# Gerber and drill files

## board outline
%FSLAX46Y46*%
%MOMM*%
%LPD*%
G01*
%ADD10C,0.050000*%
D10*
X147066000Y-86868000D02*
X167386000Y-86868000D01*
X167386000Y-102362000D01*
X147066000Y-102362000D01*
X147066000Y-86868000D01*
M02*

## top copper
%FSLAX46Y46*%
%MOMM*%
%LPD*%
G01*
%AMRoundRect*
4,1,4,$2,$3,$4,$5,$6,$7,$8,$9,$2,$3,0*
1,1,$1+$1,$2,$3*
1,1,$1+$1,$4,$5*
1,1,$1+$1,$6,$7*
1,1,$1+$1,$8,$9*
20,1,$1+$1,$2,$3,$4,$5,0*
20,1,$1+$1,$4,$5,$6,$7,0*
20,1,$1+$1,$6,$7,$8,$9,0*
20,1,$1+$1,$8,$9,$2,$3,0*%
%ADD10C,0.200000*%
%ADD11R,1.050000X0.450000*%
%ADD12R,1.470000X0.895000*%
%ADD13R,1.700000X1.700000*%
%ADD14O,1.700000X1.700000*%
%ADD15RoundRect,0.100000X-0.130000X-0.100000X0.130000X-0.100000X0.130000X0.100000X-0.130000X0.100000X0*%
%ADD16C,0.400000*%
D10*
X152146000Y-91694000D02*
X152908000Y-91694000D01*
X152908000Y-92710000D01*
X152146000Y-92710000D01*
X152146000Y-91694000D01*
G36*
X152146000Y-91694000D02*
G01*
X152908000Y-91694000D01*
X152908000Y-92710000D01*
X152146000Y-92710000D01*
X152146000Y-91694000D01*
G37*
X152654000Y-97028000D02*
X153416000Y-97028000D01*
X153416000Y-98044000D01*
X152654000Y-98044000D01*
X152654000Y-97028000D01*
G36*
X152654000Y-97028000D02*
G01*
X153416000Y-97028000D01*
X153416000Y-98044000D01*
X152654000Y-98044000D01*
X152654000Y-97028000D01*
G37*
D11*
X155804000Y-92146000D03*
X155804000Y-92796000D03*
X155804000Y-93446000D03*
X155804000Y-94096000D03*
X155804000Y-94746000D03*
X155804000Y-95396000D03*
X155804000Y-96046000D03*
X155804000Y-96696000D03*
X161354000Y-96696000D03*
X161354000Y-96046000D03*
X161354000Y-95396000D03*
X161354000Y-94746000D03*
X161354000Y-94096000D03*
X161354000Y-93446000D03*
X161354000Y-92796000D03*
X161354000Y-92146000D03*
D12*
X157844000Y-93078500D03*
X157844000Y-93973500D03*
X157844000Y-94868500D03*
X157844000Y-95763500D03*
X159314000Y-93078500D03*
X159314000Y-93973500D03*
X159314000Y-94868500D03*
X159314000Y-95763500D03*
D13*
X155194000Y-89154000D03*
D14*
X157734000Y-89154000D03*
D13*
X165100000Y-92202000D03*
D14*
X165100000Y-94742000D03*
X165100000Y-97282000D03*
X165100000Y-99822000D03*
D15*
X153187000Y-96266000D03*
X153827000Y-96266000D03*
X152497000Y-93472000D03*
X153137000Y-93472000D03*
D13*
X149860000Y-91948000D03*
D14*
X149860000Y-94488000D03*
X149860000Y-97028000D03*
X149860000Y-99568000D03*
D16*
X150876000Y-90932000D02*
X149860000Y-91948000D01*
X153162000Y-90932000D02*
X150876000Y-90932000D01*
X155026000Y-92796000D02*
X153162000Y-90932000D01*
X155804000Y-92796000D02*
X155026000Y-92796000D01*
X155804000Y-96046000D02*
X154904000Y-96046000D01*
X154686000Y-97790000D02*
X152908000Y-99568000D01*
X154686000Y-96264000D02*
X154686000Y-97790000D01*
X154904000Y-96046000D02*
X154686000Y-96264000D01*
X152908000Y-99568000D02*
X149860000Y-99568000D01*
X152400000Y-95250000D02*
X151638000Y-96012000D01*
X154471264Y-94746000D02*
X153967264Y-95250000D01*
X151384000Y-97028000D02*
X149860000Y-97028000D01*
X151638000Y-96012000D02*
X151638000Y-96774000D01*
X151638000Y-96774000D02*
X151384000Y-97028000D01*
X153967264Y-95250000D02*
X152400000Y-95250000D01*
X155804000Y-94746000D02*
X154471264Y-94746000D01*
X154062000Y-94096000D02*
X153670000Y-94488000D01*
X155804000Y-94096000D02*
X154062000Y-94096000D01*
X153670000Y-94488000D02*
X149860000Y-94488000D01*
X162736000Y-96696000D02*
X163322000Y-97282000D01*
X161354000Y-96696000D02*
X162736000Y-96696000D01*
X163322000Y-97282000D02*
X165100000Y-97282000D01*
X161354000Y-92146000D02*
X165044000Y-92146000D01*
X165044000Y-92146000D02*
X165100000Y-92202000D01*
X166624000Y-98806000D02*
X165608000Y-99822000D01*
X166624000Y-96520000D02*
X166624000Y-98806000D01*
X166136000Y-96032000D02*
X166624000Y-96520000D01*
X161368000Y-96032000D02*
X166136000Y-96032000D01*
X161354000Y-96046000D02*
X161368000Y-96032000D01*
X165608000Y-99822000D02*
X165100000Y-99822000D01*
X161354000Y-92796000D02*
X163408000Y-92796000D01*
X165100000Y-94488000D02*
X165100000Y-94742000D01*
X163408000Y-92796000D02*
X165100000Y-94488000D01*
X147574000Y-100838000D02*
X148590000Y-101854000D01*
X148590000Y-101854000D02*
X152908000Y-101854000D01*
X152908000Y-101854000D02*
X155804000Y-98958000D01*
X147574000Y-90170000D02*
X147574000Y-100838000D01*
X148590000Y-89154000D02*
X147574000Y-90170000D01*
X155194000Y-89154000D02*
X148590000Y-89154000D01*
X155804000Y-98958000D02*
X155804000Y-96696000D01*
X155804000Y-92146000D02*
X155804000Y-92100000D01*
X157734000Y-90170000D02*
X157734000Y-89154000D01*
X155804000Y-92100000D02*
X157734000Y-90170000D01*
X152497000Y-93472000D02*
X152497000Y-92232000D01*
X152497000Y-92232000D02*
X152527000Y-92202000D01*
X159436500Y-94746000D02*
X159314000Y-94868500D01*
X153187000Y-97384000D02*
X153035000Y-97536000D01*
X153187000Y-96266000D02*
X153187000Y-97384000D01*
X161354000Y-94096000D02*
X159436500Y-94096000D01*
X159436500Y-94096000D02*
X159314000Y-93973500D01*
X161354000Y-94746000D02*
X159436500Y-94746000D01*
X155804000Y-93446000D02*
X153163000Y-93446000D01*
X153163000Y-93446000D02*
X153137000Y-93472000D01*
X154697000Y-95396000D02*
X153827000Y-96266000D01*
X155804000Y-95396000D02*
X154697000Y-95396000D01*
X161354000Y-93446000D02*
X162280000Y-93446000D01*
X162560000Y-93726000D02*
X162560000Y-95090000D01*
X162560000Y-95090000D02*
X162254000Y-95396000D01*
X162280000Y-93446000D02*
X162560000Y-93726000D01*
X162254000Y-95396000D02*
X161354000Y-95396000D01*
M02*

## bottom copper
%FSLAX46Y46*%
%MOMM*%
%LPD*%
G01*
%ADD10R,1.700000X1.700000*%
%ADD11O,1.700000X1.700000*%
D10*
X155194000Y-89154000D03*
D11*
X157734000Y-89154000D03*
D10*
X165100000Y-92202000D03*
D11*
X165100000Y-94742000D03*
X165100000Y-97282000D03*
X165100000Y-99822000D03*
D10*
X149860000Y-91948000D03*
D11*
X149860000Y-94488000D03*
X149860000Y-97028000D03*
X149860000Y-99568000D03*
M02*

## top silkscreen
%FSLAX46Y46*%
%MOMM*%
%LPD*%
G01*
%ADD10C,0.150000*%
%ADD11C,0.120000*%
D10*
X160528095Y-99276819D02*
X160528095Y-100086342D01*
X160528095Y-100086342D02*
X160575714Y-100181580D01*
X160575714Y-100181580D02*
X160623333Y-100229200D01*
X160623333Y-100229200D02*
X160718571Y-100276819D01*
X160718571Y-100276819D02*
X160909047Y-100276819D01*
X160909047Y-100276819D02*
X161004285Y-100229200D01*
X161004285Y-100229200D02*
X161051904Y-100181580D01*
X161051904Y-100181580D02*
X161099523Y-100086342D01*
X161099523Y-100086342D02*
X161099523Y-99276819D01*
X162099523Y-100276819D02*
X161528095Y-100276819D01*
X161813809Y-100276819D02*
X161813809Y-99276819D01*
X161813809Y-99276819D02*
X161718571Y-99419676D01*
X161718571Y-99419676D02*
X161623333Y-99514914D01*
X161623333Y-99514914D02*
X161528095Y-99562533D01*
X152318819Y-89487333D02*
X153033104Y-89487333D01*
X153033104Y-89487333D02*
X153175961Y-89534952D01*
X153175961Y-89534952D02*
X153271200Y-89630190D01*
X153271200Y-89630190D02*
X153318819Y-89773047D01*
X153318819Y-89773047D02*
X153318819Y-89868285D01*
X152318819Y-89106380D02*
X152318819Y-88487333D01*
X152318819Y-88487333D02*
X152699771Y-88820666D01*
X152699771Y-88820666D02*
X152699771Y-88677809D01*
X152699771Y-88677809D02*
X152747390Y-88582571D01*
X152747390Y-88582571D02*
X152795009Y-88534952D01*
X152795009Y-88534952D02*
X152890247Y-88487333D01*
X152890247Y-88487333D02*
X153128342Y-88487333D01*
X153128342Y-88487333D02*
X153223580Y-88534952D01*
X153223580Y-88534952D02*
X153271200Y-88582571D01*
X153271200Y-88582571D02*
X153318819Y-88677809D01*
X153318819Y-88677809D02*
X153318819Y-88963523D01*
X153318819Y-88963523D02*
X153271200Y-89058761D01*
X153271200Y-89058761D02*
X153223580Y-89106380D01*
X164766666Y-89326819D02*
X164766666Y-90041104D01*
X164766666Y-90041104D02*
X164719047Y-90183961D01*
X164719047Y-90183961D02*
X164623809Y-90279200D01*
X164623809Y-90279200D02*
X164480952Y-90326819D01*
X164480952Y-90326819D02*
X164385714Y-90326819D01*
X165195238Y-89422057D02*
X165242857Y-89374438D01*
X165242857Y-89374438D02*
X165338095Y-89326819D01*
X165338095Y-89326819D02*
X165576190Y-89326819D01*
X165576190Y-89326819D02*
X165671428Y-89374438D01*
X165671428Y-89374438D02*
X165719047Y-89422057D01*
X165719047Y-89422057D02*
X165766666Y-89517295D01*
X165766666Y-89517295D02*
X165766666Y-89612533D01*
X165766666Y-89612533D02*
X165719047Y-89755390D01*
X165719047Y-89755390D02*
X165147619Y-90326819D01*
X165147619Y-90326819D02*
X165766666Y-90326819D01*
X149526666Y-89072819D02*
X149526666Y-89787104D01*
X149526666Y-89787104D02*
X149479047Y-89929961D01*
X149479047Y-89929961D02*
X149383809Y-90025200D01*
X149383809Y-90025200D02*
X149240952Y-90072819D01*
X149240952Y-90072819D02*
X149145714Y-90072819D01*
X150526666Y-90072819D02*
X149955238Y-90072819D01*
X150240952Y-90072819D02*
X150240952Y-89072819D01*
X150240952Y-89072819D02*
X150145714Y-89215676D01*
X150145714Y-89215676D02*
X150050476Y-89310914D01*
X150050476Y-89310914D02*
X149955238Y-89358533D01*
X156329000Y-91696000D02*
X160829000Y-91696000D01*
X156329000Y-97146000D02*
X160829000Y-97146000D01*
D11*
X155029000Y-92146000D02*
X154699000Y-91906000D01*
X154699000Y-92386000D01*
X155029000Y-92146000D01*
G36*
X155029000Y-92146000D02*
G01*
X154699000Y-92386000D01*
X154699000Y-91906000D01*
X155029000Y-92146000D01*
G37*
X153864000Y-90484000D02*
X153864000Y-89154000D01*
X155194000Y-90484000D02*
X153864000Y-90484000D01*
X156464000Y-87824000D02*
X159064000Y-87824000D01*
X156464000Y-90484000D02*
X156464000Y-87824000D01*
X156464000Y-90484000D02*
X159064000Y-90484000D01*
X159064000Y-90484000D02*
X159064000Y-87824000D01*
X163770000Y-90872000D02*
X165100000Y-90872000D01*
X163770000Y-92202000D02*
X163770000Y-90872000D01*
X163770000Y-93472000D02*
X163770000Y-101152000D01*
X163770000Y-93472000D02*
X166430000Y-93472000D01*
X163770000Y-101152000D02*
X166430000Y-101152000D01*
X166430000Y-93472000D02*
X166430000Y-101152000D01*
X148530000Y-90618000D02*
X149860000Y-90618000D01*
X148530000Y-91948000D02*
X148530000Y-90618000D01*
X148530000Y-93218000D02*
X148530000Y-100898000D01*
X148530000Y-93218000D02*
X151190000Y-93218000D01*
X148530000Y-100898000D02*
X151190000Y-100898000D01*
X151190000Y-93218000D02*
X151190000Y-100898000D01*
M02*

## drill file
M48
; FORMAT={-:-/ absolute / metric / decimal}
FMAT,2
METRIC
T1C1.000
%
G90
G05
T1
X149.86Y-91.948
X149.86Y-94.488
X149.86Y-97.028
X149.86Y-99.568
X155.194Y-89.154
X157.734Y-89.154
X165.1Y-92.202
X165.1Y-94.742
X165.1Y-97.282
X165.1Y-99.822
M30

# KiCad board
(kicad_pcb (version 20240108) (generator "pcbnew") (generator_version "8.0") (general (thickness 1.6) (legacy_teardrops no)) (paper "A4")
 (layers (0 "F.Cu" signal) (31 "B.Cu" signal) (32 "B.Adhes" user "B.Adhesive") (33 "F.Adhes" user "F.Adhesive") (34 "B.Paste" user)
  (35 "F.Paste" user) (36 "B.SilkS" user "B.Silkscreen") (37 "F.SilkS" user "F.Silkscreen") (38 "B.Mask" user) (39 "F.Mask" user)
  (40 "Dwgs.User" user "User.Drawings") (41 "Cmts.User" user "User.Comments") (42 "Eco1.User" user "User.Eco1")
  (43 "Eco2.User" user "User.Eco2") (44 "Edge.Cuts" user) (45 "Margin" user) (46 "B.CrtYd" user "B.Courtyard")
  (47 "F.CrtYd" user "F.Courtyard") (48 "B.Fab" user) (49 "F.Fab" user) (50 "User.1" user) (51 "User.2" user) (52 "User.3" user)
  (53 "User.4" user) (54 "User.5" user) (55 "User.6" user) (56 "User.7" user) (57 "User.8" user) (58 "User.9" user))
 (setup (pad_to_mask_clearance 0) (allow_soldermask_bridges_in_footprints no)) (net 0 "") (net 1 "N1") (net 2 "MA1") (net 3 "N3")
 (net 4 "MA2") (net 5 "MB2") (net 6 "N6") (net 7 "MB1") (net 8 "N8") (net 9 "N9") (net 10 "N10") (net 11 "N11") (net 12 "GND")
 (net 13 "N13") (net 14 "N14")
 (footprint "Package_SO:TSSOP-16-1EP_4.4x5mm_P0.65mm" (layer "F.Cu") (at 158.579 94.421)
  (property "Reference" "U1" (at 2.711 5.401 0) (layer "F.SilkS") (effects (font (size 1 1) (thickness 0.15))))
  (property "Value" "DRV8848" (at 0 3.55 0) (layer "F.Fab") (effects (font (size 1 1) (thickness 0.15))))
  (fp_line (start -2.25 -2.725) (end 2.25 -2.725) (stroke (width 0.15) (type solid)) (layer "F.SilkS"))
  (fp_line (start -2.25 2.725) (end 2.25 2.725) (stroke (width 0.15) (type solid)) (layer "F.SilkS"))
  (fp_poly
   (pts (xy -3.55 -2.275) (xy -3.88 -2.515) (xy -3.88 -2.035) (xy -3.55 -2.275)) (stroke (width 0.12) (type solid)) (fill solid)
   (layer "F.SilkS"))
  (pad "1" smd rect (at -2.775 -2.275) (size 1.05 0.45) (layers "F.Cu" "F.Paste" "F.Mask") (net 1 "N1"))
  (pad "2" smd rect (at -2.775 -1.625) (size 1.05 0.45) (layers "F.Cu" "F.Paste" "F.Mask") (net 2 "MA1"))
  (pad "3" smd rect (at -2.775 -0.975) (size 1.05 0.45) (layers "F.Cu" "F.Paste" "F.Mask") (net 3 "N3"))
  (pad "4" smd rect (at -2.775 -0.325) (size 1.05 0.45) (layers "F.Cu" "F.Paste" "F.Mask") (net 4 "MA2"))
  (pad "5" smd rect (at -2.775 0.325) (size 1.05 0.45) (layers "F.Cu" "F.Paste" "F.Mask") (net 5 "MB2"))
  (pad "6" smd rect (at -2.775 0.975) (size 1.05 0.45) (layers "F.Cu" "F.Paste" "F.Mask") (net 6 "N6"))
  (pad "7" smd rect (at -2.775 1.625) (size 1.05 0.45) (layers "F.Cu" "F.Paste" "F.Mask") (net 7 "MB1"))
  (pad "8" smd rect (at -2.775 2.275) (size 1.05 0.45) (layers "F.Cu" "F.Paste" "F.Mask") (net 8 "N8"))
  (pad "9" smd rect (at 2.775 2.275) (size 1.05 0.45) (layers "F.Cu" "F.Paste" "F.Mask") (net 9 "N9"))
  (pad "10" smd rect (at 2.775 1.625) (size 1.05 0.45) (layers "F.Cu" "F.Paste" "F.Mask") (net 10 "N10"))
  (pad "11" smd rect (at 2.775 0.975) (size 1.05 0.45) (layers "F.Cu" "F.Paste" "F.Mask") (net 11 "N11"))
  (pad "12" smd rect (at 2.775 0.325) (size 1.05 0.45) (layers "F.Cu" "F.Paste" "F.Mask") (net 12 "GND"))
  (pad "13" smd rect (at 2.775 -0.325) (size 1.05 0.45) (layers "F.Cu" "F.Paste" "F.Mask") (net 12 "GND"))
  (pad "14" smd rect (at 2.775 -0.975) (size 1.05 0.45) (layers "F.Cu" "F.Paste" "F.Mask") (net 11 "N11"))
  (pad "15" smd rect (at 2.775 -1.625) (size 1.05 0.45) (layers "F.Cu" "F.Paste" "F.Mask") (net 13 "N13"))
  (pad "16" smd rect (at 2.775 -2.275) (size 1.05 0.45) (layers "F.Cu" "F.Paste" "F.Mask") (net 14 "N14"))
  (pad "17" smd rect (at -0.735 -1.3425) (size 1.47 0.895) (layers "F.Cu" "F.Paste" "F.Mask") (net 12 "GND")
   (solder_paste_margin_ratio -0.2))
  (pad "17" smd rect (at -0.735 -0.4475) (size 1.47 0.895) (layers "F.Cu" "F.Paste" "F.Mask") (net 12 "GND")
   (solder_paste_margin_ratio -0.2))
  (pad "17" smd rect (at -0.735 0.4475) (size 1.47 0.895) (layers "F.Cu" "F.Paste" "F.Mask") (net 12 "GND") (solder_paste_margin_ratio -0.2))
  (pad "17" smd rect (at -0.735 1.3425) (size 1.47 0.895) (layers "F.Cu" "F.Paste" "F.Mask") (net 12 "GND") (solder_paste_margin_ratio -0.2))
  (pad "17" smd rect (at 0.735 -1.3425) (size 1.47 0.895) (layers "F.Cu" "F.Paste" "F.Mask") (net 12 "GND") (solder_paste_margin_ratio -0.2))
  (pad "17" smd rect (at 0.735 -0.4475) (size 1.47 0.895) (layers "F.Cu" "F.Paste" "F.Mask") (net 12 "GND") (solder_paste_margin_ratio -0.2))
  (pad "17" smd rect (at 0.735 0.4475) (size 1.47 0.895) (layers "F.Cu" "F.Paste" "F.Mask") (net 12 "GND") (solder_paste_margin_ratio -0.2))
  (pad "17" smd rect (at 0.735 1.3425) (size 1.47 0.895) (layers "F.Cu" "F.Paste" "F.Mask") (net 12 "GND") (solder_paste_margin_ratio -0.2)))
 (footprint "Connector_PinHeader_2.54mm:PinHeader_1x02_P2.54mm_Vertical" (layer "F.Cu") (at 155.194 89.154 90)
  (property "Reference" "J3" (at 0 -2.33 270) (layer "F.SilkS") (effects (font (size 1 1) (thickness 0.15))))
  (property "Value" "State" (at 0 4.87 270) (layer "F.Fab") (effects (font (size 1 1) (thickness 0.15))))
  (fp_line (start -1.33 -1.33) (end 0 -1.33) (stroke (width 0.12) (type solid)) (layer "F.SilkS"))
  (fp_line (start -1.33 0) (end -1.33 -1.33) (stroke (width 0.12) (type solid)) (layer "F.SilkS"))
  (fp_line (start 1.33 1.27) (end 1.33 3.87) (stroke (width 0.12) (type solid)) (layer "F.SilkS"))
  (fp_line (start -1.33 1.27) (end 1.33 1.27) (stroke (width 0.12) (type solid)) (layer "F.SilkS"))
  (fp_line (start -1.33 1.27) (end -1.33 3.87) (stroke (width 0.12) (type solid)) (layer "F.SilkS"))
  (fp_line (start -1.33 3.87) (end 1.33 3.87) (stroke (width 0.12) (type solid)) (layer "F.SilkS"))
  (pad "1" thru_hole rect (at 0 0 90) (size 1.7 1.7) (drill 1) (layers "*.Cu" "*.Mask") (remove_unused_layers no) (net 8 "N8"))
  (pad "2" thru_hole oval (at 0 2.54 90) (size 1.7 1.7) (drill 1) (layers "*.Cu" "*.Mask") (remove_unused_layers no) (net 1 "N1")))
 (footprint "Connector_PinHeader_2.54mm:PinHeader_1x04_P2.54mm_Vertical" (layer "F.Cu") (at 165.1 92.202)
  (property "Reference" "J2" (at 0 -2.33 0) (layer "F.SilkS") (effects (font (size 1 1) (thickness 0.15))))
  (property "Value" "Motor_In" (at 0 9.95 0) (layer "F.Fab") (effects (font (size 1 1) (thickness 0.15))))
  (fp_line (start -1.33 -1.33) (end 0 -1.33) (stroke (width 0.12) (type solid)) (layer "F.SilkS"))
  (fp_line (start -1.33 0) (end -1.33 -1.33) (stroke (width 0.12) (type solid)) (layer "F.SilkS"))
  (fp_line (start -1.33 1.27) (end -1.33 8.95) (stroke (width 0.12) (type solid)) (layer "F.SilkS"))
  (fp_line (start -1.33 1.27) (end 1.33 1.27) (stroke (width 0.12) (type solid)) (layer "F.SilkS"))
  (fp_line (start -1.33 8.95) (end 1.33 8.95) (stroke (width 0.12) (type solid)) (layer "F.SilkS"))
  (fp_line (start 1.33 1.27) (end 1.33 8.95) (stroke (width 0.12) (type solid)) (layer "F.SilkS"))
  (pad "1" thru_hole rect (at 0 0) (size 1.7 1.7) (drill 1) (layers "*.Cu" "*.Mask") (remove_unused_layers no) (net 14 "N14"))
  (pad "2" thru_hole oval (at 0 2.54) (size 1.7 1.7) (drill 1) (layers "*.Cu" "*.Mask") (remove_unused_layers no) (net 13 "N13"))
  (pad "3" thru_hole oval (at 0 5.08) (size 1.7 1.7) (drill 1) (layers "*.Cu" "*.Mask") (remove_unused_layers no) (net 9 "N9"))
  (pad "4" thru_hole oval (at 0 7.62) (size 1.7 1.7) (drill 1) (layers "*.Cu" "*.Mask") (remove_unused_layers no) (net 10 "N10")))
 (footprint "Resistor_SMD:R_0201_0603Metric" (layer "F.Cu") (at 153.507 96.266)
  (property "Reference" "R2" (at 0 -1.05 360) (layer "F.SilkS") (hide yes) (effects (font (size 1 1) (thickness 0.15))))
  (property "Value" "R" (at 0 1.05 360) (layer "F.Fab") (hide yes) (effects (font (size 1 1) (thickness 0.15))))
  (pad "" smd roundrect (at -0.345 0) (size 0.318 0.36) (layers "F.Paste") (roundrect_rratio 0.25))
  (pad "" smd roundrect (at 0.345 0) (size 0.318 0.36) (layers "F.Paste") (roundrect_rratio 0.25))
  (pad "1" smd roundrect (at -0.32 0) (size 0.46 0.4) (layers "F.Cu" "F.Mask") (roundrect_rratio 0.25) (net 12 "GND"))
  (pad "2" smd roundrect (at 0.32 0) (size 0.46 0.4) (layers "F.Cu" "F.Mask") (roundrect_rratio 0.25) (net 6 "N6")))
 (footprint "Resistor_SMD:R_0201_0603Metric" (layer "F.Cu") (at 152.817 93.472)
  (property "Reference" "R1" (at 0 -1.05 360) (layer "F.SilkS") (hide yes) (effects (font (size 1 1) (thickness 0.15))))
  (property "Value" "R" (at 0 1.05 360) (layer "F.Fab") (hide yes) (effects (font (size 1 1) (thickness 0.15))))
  (pad "" smd roundrect (at -0.345 0) (size 0.318 0.36) (layers "F.Paste") (roundrect_rratio 0.25))
  (pad "" smd roundrect (at 0.345 0) (size 0.318 0.36) (layers "F.Paste") (roundrect_rratio 0.25))
  (pad "1" smd roundrect (at -0.32 0) (size 0.46 0.4) (layers "F.Cu" "F.Mask") (roundrect_rratio 0.25) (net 12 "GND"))
  (pad "2" smd roundrect (at 0.32 0) (size 0.46 0.4) (layers "F.Cu" "F.Mask") (roundrect_rratio 0.25) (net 3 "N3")))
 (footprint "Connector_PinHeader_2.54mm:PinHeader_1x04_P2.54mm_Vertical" (layer "F.Cu") (at 149.86 91.948)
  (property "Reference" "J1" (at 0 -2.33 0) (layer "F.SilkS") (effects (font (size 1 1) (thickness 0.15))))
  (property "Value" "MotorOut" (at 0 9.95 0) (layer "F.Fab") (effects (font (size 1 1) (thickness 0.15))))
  (fp_line (start -1.33 -1.33) (end 0 -1.33) (stroke (width 0.12) (type solid)) (layer "F.SilkS"))
  (fp_line (start -1.33 0) (end -1.33 -1.33) (stroke (width 0.12) (type solid)) (layer "F.SilkS"))
  (fp_line (start -1.33 1.27) (end -1.33 8.95) (stroke (width 0.12) (type solid)) (layer "F.SilkS"))
  (fp_line (start -1.33 1.27) (end 1.33 1.27) (stroke (width 0.12) (type solid)) (layer "F.SilkS"))
  (fp_line (start -1.33 8.95) (end 1.33 8.95) (stroke (width 0.12) (type solid)) (layer "F.SilkS"))
  (fp_line (start 1.33 1.27) (end 1.33 8.95) (stroke (width 0.12) (type solid)) (layer "F.SilkS"))
  (pad "1" thru_hole rect (at 0 0) (size 1.7 1.7) (drill 1) (layers "*.Cu" "*.Mask") (remove_unused_layers no) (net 2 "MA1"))
  (pad "2" thru_hole oval (at 0 2.54) (size 1.7 1.7) (drill 1) (layers "*.Cu" "*.Mask") (remove_unused_layers no) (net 4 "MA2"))
  (pad "3" thru_hole oval (at 0 5.08) (size 1.7 1.7) (drill 1) (layers "*.Cu" "*.Mask") (remove_unused_layers no) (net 5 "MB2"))
  (pad "4" thru_hole oval (at 0 7.62) (size 1.7 1.7) (drill 1) (layers "*.Cu" "*.Mask") (remove_unused_layers no) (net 7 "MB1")))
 (gr_rect (start 152.146 91.694) (end 152.908 92.71) (stroke (width 0.2) (type default)) (fill solid) (layer "F.Cu") (net 12))
 (gr_rect (start 152.654 97.028) (end 153.416 98.044) (stroke (width 0.2) (type default)) (fill solid) (layer "F.Cu") (net 12))
 (gr_rect (start 147.066 86.868) (end 167.386 102.362) (stroke (width 0.05) (type default)) (fill none) (layer "Edge.Cuts"))
 (segment (start 150.876 90.932) (end 149.86 91.948) (width 0.4) (layer "F.Cu") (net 2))
 (segment (start 153.162 90.932) (end 150.876 90.932) (width 0.4) (layer "F.Cu") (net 2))
 (segment (start 155.026 92.796) (end 153.162 90.932) (width 0.4) (layer "F.Cu") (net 2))
 (segment (start 155.804 92.796) (end 155.026 92.796) (width 0.4) (layer "F.Cu") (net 2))
 (segment (start 155.804 96.046) (end 154.904 96.046) (width 0.4) (layer "F.Cu") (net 7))
 (segment (start 154.686 97.79) (end 152.908 99.568) (width 0.4) (layer "F.Cu") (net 7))
 (segment (start 154.686 96.264) (end 154.686 97.79) (width 0.4) (layer "F.Cu") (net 7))
 (segment (start 154.904 96.046) (end 154.686 96.264) (width 0.4) (layer "F.Cu") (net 7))
 (segment (start 152.908 99.568) (end 149.86 99.568) (width 0.4) (layer "F.Cu") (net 7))
 (segment (start 152.4 95.25) (end 151.638 96.012) (width 0.4) (layer "F.Cu") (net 5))
 (segment (start 154.471264 94.746) (end 153.967264 95.25) (width 0.4) (layer "F.Cu") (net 5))
 (segment (start 151.384 97.028) (end 149.86 97.028) (width 0.4) (layer "F.Cu") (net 5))
 (segment (start 151.638 96.012) (end 151.638 96.774) (width 0.4) (layer "F.Cu") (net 5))
 (segment (start 151.638 96.774) (end 151.384 97.028) (width 0.4) (layer "F.Cu") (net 5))
 (segment (start 153.967264 95.25) (end 152.4 95.25) (width 0.4) (layer "F.Cu") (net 5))
 (segment (start 155.804 94.746) (end 154.471264 94.746) (width 0.4) (layer "F.Cu") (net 5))
 (segment (start 154.062 94.096) (end 153.67 94.488) (width 0.4) (layer "F.Cu") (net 4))
 (segment (start 155.804 94.096) (end 154.062 94.096) (width 0.4) (layer "F.Cu") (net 4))
 (segment (start 153.67 94.488) (end 149.86 94.488) (width 0.4) (layer "F.Cu") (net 4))
 (segment (start 162.736 96.696) (end 163.322 97.282) (width 0.4) (layer "F.Cu") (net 9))
 (segment (start 161.354 96.696) (end 162.736 96.696) (width 0.4) (layer "F.Cu") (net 9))
 (segment (start 163.322 97.282) (end 165.1 97.282) (width 0.4) (layer "F.Cu") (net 9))
 (segment (start 161.354 92.146) (end 165.044 92.146) (width 0.4) (layer "F.Cu") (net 14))
 (segment (start 165.044 92.146) (end 165.1 92.202) (width 0.4) (layer "F.Cu") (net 14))
 (segment (start 166.624 98.806) (end 165.608 99.822) (width 0.4) (layer "F.Cu") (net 10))
 (segment (start 166.624 96.52) (end 166.624 98.806) (width 0.4) (layer "F.Cu") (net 10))
 (segment (start 166.136 96.032) (end 166.624 96.52) (width 0.4) (layer "F.Cu") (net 10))
 (segment (start 161.368 96.032) (end 166.136 96.032) (width 0.4) (layer "F.Cu") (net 10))
 (segment (start 161.354 96.046) (end 161.368 96.032) (width 0.4) (layer "F.Cu") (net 10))
 (segment (start 165.608 99.822) (end 165.1 99.822) (width 0.4) (layer "F.Cu") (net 10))
 (segment (start 161.354 92.796) (end 163.408 92.796) (width 0.4) (layer "F.Cu") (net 13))
 (segment (start 165.1 94.488) (end 165.1 94.742) (width 0.4) (layer "F.Cu") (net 13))
 (segment (start 163.408 92.796) (end 165.1 94.488) (width 0.4) (layer "F.Cu") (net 13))
 (segment (start 147.574 100.838) (end 148.59 101.854) (width 0.4) (layer "F.Cu") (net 8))
 (segment (start 148.59 101.854) (end 152.908 101.854) (width 0.4) (layer "F.Cu") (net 8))
 (segment (start 152.908 101.854) (end 155.804 98.958) (width 0.4) (layer "F.Cu") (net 8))
 (segment (start 147.574 90.17) (end 147.574 100.838) (width 0.4) (layer "F.Cu") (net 8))
 (segment (start 148.59 89.154) (end 147.574 90.17) (width 0.4) (layer "F.Cu") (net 8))
 (segment (start 155.194 89.154) (end 148.59 89.154) (width 0.4) (layer "F.Cu") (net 8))
 (segment (start 155.804 98.958) (end 155.804 96.696) (width 0.4) (layer "F.Cu") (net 8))
 (segment (start 155.804 92.146) (end 155.804 92.1) (width 0.4) (layer "F.Cu") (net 1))
 (segment (start 157.734 90.17) (end 157.734 89.154) (width 0.4) (layer "F.Cu") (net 1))
 (segment (start 155.804 92.1) (end 157.734 90.17) (width 0.4) (layer "F.Cu") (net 1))
 (segment (start 152.497 93.472) (end 152.497 92.232) (width 0.4) (layer "F.Cu") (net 12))
 (segment (start 152.497 92.232) (end 152.527 92.202) (width 0.4) (layer "F.Cu") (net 12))
 (segment (start 159.4365 94.746) (end 159.314 94.8685) (width 0.4) (layer "F.Cu") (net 12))
 (segment (start 153.187 97.384) (end 153.035 97.536) (width 0.4) (layer "F.Cu") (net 12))
 (segment (start 153.187 96.266) (end 153.187 97.384) (width 0.4) (layer "F.Cu") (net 12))
 (segment (start 161.354 94.096) (end 159.4365 94.096) (width 0.4) (layer "F.Cu") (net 12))
 (segment (start 159.4365 94.096) (end 159.314 93.9735) (width 0.4) (layer "F.Cu") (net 12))
 (segment (start 161.354 94.746) (end 159.4365 94.746) (width 0.4) (layer "F.Cu") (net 12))
 (segment (start 155.804 93.446) (end 153.163 93.446) (width 0.4) (layer "F.Cu") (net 3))
 (segment (start 153.163 93.446) (end 153.137 93.472) (width 0.4) (layer "F.Cu") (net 3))
 (segment (start 154.697 95.396) (end 153.827 96.266) (width 0.4) (layer "F.Cu") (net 6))
 (segment (start 155.804 95.396) (end 154.697 95.396) (width 0.4) (layer "F.Cu") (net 6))
 (segment (start 161.354 93.446) (end 162.28 93.446) (width 0.4) (layer "F.Cu") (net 11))
 (segment (start 162.56 93.726) (end 162.56 95.09) (width 0.4) (layer "F.Cu") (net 11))
 (segment (start 162.56 95.09) (end 162.254 95.396) (width 0.4) (layer "F.Cu") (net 11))
 (segment (start 162.28 93.446) (end 162.56 93.726) (width 0.4) (layer "F.Cu") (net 11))
 (segment (start 162.254 95.396) (end 161.354 95.396) (width 0.4) (layer "F.Cu") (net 11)))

